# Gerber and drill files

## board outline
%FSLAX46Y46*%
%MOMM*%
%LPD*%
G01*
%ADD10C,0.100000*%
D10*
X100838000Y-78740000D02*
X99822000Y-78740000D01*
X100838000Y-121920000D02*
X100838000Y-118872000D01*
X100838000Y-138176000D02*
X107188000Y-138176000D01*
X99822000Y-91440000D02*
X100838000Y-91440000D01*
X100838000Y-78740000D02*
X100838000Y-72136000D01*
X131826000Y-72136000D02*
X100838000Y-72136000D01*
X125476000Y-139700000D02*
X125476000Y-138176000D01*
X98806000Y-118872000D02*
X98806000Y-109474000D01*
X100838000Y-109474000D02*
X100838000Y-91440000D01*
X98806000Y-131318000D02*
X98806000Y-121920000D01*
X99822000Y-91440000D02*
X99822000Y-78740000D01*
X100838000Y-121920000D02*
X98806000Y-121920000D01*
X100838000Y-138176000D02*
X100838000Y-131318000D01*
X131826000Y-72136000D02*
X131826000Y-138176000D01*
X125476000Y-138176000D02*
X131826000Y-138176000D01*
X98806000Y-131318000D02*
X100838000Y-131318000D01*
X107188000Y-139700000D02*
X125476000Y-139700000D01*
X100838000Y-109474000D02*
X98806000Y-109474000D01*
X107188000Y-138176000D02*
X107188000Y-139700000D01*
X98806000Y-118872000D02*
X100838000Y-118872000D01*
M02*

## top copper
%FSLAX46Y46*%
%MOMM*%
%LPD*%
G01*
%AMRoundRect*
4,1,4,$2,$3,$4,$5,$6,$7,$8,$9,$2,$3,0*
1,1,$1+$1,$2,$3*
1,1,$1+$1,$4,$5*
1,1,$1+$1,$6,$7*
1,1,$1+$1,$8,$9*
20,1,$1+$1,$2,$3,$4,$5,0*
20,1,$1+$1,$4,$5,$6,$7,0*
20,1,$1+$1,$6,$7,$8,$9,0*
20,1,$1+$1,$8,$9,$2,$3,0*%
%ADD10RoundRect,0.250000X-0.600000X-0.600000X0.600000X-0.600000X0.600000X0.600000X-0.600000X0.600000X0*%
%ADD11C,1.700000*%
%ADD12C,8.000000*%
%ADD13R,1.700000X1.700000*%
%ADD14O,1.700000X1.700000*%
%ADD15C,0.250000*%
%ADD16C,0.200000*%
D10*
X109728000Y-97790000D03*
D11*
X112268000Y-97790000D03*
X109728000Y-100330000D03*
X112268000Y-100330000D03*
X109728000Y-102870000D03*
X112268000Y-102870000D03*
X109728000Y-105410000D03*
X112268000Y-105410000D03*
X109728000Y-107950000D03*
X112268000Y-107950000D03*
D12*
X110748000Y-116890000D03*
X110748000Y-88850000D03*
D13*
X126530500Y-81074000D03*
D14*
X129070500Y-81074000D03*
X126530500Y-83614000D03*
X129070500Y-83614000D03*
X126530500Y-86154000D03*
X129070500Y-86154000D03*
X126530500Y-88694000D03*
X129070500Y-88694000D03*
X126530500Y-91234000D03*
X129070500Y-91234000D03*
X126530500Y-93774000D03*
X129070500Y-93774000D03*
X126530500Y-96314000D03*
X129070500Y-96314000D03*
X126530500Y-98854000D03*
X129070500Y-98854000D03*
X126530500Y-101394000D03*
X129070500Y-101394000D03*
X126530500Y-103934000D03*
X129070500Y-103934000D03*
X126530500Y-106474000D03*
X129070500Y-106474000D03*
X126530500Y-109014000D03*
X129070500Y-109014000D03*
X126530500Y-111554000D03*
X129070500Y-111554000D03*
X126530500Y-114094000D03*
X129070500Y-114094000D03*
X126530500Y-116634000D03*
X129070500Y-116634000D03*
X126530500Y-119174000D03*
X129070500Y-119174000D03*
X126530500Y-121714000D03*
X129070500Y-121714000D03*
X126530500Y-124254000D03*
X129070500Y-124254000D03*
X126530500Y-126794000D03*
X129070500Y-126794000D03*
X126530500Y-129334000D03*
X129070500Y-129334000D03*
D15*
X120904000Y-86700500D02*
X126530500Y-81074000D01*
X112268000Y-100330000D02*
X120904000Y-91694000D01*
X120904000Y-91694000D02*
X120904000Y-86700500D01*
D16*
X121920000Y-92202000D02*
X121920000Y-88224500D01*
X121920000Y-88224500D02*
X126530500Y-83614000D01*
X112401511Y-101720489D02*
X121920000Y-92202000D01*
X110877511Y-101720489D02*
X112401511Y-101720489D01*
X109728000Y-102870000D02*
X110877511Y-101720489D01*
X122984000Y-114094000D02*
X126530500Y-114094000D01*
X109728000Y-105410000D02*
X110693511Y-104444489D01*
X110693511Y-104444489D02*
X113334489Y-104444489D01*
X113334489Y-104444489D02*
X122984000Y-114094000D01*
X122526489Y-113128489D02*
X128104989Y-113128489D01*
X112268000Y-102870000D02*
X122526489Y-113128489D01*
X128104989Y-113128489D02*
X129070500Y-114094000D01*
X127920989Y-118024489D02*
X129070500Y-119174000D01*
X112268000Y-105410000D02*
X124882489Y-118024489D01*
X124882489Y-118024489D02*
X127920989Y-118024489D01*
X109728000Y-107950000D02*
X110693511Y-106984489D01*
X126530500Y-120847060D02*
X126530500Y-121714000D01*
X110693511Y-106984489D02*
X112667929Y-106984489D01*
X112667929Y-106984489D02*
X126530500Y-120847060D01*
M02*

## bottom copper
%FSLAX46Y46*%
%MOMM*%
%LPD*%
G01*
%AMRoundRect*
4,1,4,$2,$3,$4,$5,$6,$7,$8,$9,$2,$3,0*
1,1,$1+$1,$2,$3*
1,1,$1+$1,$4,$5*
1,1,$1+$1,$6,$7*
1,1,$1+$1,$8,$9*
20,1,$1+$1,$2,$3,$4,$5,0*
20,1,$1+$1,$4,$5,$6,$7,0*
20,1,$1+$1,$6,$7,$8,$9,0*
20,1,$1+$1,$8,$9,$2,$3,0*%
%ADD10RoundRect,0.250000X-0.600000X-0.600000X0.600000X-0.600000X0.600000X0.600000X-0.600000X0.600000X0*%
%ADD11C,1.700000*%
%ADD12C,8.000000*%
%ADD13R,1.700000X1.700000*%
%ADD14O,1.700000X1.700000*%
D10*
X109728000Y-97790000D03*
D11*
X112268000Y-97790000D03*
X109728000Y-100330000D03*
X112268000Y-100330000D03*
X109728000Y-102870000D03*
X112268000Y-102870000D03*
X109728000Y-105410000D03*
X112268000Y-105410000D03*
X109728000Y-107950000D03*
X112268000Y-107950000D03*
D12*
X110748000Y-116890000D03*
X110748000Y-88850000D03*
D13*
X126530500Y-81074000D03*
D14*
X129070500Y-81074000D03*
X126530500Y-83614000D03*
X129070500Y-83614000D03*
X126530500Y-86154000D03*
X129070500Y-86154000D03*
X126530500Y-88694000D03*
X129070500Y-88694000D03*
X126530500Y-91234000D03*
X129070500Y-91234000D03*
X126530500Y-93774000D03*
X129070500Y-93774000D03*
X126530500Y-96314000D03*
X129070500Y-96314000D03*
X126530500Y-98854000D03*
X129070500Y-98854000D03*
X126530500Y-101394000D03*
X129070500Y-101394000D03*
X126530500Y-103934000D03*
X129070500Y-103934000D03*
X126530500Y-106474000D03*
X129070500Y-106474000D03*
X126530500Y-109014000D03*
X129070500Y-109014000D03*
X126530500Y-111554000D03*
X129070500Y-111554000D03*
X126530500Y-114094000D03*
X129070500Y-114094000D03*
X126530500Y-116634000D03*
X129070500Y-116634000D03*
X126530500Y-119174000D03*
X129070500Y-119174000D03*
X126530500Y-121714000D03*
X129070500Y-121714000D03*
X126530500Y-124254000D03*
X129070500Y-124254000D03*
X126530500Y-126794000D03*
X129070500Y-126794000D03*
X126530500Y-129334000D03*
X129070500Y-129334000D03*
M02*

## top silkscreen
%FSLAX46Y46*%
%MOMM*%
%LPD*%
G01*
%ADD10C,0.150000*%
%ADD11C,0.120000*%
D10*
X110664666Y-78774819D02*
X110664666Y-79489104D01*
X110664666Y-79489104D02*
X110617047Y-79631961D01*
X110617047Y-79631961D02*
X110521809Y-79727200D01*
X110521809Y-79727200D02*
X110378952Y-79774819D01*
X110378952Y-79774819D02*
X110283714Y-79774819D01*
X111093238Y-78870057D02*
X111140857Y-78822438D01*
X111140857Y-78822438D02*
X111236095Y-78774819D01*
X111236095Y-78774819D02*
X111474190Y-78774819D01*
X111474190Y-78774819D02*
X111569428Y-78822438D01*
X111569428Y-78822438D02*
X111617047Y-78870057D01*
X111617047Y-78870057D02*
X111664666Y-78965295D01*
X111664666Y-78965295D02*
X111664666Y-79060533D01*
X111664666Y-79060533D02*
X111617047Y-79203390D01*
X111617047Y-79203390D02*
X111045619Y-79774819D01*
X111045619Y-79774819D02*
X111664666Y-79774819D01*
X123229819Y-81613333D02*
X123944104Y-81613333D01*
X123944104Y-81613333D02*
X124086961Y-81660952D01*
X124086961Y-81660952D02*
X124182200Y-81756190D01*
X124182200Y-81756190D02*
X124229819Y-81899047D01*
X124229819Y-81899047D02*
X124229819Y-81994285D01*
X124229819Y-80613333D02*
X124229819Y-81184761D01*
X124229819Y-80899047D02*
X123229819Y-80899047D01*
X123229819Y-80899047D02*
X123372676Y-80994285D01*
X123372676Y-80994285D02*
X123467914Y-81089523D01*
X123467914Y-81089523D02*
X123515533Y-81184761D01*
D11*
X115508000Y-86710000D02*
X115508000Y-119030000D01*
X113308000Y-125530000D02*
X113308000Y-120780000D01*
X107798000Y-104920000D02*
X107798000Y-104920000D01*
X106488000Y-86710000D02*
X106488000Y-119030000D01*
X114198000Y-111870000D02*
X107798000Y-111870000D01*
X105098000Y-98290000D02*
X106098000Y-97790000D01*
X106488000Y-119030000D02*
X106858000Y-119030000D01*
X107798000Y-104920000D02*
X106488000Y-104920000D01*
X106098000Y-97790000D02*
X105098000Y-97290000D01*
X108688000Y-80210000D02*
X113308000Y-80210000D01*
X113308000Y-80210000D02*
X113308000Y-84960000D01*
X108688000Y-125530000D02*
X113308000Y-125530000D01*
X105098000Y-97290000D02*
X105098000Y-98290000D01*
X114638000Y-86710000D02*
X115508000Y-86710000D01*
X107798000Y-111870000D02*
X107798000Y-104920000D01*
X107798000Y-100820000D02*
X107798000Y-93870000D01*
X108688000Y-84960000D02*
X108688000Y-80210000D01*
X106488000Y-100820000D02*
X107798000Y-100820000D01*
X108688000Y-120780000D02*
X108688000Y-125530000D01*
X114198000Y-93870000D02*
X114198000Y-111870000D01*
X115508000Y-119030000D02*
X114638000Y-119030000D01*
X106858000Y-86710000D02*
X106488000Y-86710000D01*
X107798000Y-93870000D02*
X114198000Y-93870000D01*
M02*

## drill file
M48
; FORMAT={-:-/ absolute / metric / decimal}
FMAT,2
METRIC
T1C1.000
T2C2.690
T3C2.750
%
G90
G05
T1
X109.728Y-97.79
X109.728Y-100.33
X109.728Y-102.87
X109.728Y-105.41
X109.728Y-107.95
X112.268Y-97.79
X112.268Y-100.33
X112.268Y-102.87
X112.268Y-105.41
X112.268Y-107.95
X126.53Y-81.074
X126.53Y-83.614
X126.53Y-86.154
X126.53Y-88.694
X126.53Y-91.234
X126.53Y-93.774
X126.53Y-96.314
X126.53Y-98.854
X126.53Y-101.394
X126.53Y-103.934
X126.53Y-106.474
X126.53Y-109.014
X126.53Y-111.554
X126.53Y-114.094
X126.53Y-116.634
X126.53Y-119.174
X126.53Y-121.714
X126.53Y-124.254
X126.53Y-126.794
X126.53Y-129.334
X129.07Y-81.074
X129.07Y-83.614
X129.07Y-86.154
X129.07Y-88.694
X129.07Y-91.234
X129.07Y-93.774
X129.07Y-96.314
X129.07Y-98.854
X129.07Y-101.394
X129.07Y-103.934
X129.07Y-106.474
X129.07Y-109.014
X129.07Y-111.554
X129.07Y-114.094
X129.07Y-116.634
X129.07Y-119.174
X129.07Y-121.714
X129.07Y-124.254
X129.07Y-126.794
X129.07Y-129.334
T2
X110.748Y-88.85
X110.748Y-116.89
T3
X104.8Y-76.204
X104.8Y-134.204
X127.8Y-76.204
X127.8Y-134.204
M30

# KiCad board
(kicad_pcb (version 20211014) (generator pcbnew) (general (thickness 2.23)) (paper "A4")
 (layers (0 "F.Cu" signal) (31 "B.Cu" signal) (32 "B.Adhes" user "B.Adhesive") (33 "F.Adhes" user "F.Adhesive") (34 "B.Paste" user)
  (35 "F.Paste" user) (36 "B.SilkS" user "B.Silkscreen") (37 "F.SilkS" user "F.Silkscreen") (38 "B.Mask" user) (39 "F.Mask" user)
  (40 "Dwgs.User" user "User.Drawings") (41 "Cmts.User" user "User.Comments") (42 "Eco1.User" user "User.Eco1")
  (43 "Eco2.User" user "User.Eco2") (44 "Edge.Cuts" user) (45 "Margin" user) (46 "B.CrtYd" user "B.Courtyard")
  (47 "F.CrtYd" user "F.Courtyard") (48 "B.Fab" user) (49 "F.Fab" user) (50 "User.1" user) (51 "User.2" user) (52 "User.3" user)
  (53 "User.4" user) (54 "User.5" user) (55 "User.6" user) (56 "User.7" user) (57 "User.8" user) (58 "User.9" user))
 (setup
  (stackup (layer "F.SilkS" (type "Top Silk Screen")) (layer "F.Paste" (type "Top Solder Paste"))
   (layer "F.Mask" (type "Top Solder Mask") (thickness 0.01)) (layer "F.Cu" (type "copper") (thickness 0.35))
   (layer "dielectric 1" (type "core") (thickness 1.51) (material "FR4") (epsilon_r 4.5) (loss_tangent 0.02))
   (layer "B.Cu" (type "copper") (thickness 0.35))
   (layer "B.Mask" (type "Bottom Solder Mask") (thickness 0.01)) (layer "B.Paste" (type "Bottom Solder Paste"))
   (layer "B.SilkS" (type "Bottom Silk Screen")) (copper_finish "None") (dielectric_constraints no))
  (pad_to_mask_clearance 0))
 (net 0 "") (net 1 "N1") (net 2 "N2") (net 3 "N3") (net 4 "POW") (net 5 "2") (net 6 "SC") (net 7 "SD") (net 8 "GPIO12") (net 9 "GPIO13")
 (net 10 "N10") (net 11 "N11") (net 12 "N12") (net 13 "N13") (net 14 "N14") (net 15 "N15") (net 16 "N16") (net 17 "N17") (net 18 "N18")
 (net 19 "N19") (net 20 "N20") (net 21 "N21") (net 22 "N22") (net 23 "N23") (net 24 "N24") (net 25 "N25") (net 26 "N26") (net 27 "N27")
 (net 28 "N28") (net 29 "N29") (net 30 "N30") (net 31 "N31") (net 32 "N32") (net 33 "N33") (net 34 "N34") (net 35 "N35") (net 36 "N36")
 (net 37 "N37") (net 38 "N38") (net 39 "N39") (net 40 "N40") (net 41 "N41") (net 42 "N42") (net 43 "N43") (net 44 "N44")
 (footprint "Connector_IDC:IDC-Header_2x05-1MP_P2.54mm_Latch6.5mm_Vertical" (layer "F.Cu") (at 109.728 97.79)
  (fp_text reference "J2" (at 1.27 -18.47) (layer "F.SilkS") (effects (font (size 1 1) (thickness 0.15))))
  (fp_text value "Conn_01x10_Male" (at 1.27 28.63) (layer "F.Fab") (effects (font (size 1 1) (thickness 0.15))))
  (fp_line (start 5.78 -11.08) (end 5.78 21.24) (layer "F.SilkS") (width 0.12))
  (fp_line (start 3.58 27.74) (end 3.58 22.99) (layer "F.SilkS") (width 0.12))
  (fp_line (start -1.93 7.13) (end -1.93 7.13) (layer "F.SilkS") (width 0.12))
  (fp_line (start -3.24 -11.08) (end -3.24 21.24) (layer "F.SilkS") (width 0.12))
  (fp_line (start 4.47 14.08) (end -1.93 14.08) (layer "F.SilkS") (width 0.12))
  (fp_line (start -4.63 0.5) (end -3.63 0) (layer "F.SilkS") (width 0.12))
  (fp_line (start -3.24 21.24) (end -2.87 21.24) (layer "F.SilkS") (width 0.12))
  (fp_line (start -1.93 7.13) (end -3.24 7.13) (layer "F.SilkS") (width 0.12))
  (fp_line (start -3.63 0) (end -4.63 -0.5) (layer "F.SilkS") (width 0.12))
  (fp_line (start -1.04 -17.58) (end 3.58 -17.58) (layer "F.SilkS") (width 0.12))
  (fp_line (start 3.58 -17.58) (end 3.58 -12.83) (layer "F.SilkS") (width 0.12))
  (fp_line (start -1.04 27.74) (end 3.58 27.74) (layer "F.SilkS") (width 0.12))
  (fp_line (start -4.63 -0.5) (end -4.63 0.5) (layer "F.SilkS") (width 0.12))
  (fp_line (start 4.91 -11.08) (end 5.78 -11.08) (layer "F.SilkS") (width 0.12))
  (fp_line (start -1.93 14.08) (end -1.93 7.13) (layer "F.SilkS") (width 0.12))
  (fp_line (start -1.93 3.03) (end -1.93 -3.92) (layer "F.SilkS") (width 0.12))
  (fp_line (start -1.04 -12.83) (end -1.04 -17.58) (layer "F.SilkS") (width 0.12))
  (fp_line (start -3.24 3.03) (end -1.93 3.03) (layer "F.SilkS") (width 0.12))
  (fp_line (start -1.04 22.99) (end -1.04 27.74) (layer "F.SilkS") (width 0.12))
  (fp_line (start 4.47 -3.92) (end 4.47 14.08) (layer "F.SilkS") (width 0.12))
  (fp_line (start 5.78 21.24) (end 4.91 21.24) (layer "F.SilkS") (width 0.12))
  (fp_line (start -2.87 -11.08) (end -3.24 -11.08) (layer "F.SilkS") (width 0.12))
  (fp_line (start -1.93 -3.92) (end 4.47 -3.92) (layer "F.SilkS") (width 0.12))
  (pad "1" thru_hole roundrect (at 0 0) (size 1.7 1.7) (drill 1) (layers *.Cu *.Mask) (roundrect_rratio 0.147059) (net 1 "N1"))
  (pad "2" thru_hole circle (at 2.54 0) (size 1.7 1.7) (drill 1) (layers *.Cu *.Mask) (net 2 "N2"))
  (pad "3" thru_hole circle (at 0 2.54) (size 1.7 1.7) (drill 1) (layers *.Cu *.Mask) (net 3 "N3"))
  (pad "4" thru_hole circle (at 2.54 2.54) (size 1.7 1.7) (drill 1) (layers *.Cu *.Mask) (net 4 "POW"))
  (pad "5" thru_hole circle (at 0 5.08) (size 1.7 1.7) (drill 1) (layers *.Cu *.Mask) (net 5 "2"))
  (pad "6" thru_hole circle (at 2.54 5.08) (size 1.7 1.7) (drill 1) (layers *.Cu *.Mask) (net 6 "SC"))
  (pad "7" thru_hole circle (at 0 7.62) (size 1.7 1.7) (drill 1) (layers *.Cu *.Mask) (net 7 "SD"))
  (pad "8" thru_hole circle (at 2.54 7.62) (size 1.7 1.7) (drill 1) (layers *.Cu *.Mask) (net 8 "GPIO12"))
  (pad "9" thru_hole circle (at 0 10.16) (size 1.7 1.7) (drill 1) (layers *.Cu *.Mask) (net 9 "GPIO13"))
  (pad "10" thru_hole circle (at 2.54 10.16) (size 1.7 1.7) (drill 1) (layers *.Cu *.Mask) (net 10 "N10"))
  (pad "MP" thru_hole circle (at 1.02 19.1) (size 8 8) (drill 2.69) (layers *.Cu *.Mask))
  (pad "MP" thru_hole circle (at 1.02 -8.94) (size 8 8) (drill 2.69) (layers *.Cu *.Mask)))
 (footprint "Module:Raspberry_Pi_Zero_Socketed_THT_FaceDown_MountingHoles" (layer "B.Cu") (at 126.5305 81.074 180)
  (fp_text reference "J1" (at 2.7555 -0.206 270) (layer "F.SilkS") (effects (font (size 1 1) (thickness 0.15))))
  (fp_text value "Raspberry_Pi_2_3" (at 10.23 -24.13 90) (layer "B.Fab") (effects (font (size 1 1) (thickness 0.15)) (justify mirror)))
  (pad "" np_thru_hole circle (at 21.73 4.87 90) (size 2.75 2.75) (drill 2.75) (layers *.Cu *.Mask) (solder_mask_margin 1.625))
  (pad "" np_thru_hole circle (at 21.73 -53.13 90) (size 2.75 2.75) (drill 2.75) (layers *.Cu *.Mask) (solder_mask_margin 1.625))
  (pad "" np_thru_hole circle (at -1.27 4.87 90) (size 2.75 2.75) (drill 2.75) (layers *.Cu *.Mask) (solder_mask_margin 1.625))
  (pad "" np_thru_hole circle (at -1.27 -53.13 90) (size 2.75 2.75) (drill 2.75) (layers *.Cu *.Mask) (solder_mask_margin 1.625))
  (pad "1" thru_hole rect (at 0 0 180) (size 1.7 1.7) (drill 1) (layers *.Cu *.Mask) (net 4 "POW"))
  (pad "2" thru_hole oval (at -2.54 0 180) (size 1.7 1.7) (drill 1) (layers *.Cu *.Mask) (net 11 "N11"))
  (pad "3" thru_hole oval (at 0 -2.54 180) (size 1.7 1.7) (drill 1) (layers *.Cu *.Mask) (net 5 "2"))
  (pad "4" thru_hole oval (at -2.54 -2.54 180) (size 1.7 1.7) (drill 1) (layers *.Cu *.Mask) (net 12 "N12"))
  (pad "5" thru_hole oval (at 0 -5.08 180) (size 1.7 1.7) (drill 1) (layers *.Cu *.Mask) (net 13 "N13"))
  (pad "6" thru_hole oval (at -2.54 -5.08 180) (size 1.7 1.7) (drill 1) (layers *.Cu *.Mask) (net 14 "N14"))
  (pad "7" thru_hole oval (at 0 -7.62 180) (size 1.7 1.7) (drill 1) (layers *.Cu *.Mask) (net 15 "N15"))
  (pad "8" thru_hole oval (at -2.54 -7.62 180) (size 1.7 1.7) (drill 1) (layers *.Cu *.Mask) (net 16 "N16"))
  (pad "9" thru_hole oval (at 0 -10.16 180) (size 1.7 1.7) (drill 1) (layers *.Cu *.Mask) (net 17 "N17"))
  (pad "10" thru_hole oval (at -2.54 -10.16 180) (size 1.7 1.7) (drill 1) (layers *.Cu *.Mask) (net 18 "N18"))
  (pad "11" thru_hole oval (at 0 -12.7 180) (size 1.7 1.7) (drill 1) (layers *.Cu *.Mask) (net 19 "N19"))
  (pad "12" thru_hole oval (at -2.54 -12.7 180) (size 1.7 1.7) (drill 1) (layers *.Cu *.Mask) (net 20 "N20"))
  (pad "13" thru_hole oval (at 0 -15.24 180) (size 1.7 1.7) (drill 1) (layers *.Cu *.Mask) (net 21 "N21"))
  (pad "14" thru_hole oval (at -2.54 -15.24 180) (size 1.7 1.7) (drill 1) (layers *.Cu *.Mask) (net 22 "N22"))
  (pad "15" thru_hole oval (at 0 -17.78 180) (size 1.7 1.7) (drill 1) (layers *.Cu *.Mask) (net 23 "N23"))
  (pad "16" thru_hole oval (at -2.54 -17.78 180) (size 1.7 1.7) (drill 1) (layers *.Cu *.Mask) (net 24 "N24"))
  (pad "17" thru_hole oval (at 0 -20.32 180) (size 1.7 1.7) (drill 1) (layers *.Cu *.Mask) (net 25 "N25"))
  (pad "18" thru_hole oval (at -2.54 -20.32 180) (size 1.7 1.7) (drill 1) (layers *.Cu *.Mask) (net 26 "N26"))
  (pad "19" thru_hole oval (at 0 -22.86 180) (size 1.7 1.7) (drill 1) (layers *.Cu *.Mask) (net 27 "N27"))
  (pad "20" thru_hole oval (at -2.54 -22.86 180) (size 1.7 1.7) (drill 1) (layers *.Cu *.Mask) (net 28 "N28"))
  (pad "21" thru_hole oval (at 0 -25.4 180) (size 1.7 1.7) (drill 1) (layers *.Cu *.Mask) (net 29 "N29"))
  (pad "22" thru_hole oval (at -2.54 -25.4 180) (size 1.7 1.7) (drill 1) (layers *.Cu *.Mask) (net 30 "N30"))
  (pad "23" thru_hole oval (at 0 -27.94 180) (size 1.7 1.7) (drill 1) (layers *.Cu *.Mask) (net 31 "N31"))
  (pad "24" thru_hole oval (at -2.54 -27.94 180) (size 1.7 1.7) (drill 1) (layers *.Cu *.Mask) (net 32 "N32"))
  (pad "25" thru_hole oval (at 0 -30.48 180) (size 1.7 1.7) (drill 1) (layers *.Cu *.Mask) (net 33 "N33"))
  (pad "26" thru_hole oval (at -2.54 -30.48 180) (size 1.7 1.7) (drill 1) (layers *.Cu *.Mask) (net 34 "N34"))
  (pad "27" thru_hole oval (at 0 -33.02 180) (size 1.7 1.7) (drill 1) (layers *.Cu *.Mask) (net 7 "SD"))
  (pad "28" thru_hole oval (at -2.54 -33.02 180) (size 1.7 1.7) (drill 1) (layers *.Cu *.Mask) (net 6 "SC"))
  (pad "29" thru_hole oval (at 0 -35.56 180) (size 1.7 1.7) (drill 1) (layers *.Cu *.Mask) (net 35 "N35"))
  (pad "30" thru_hole oval (at -2.54 -35.56 180) (size 1.7 1.7) (drill 1) (layers *.Cu *.Mask) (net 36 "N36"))
  (pad "31" thru_hole oval (at 0 -38.1 180) (size 1.7 1.7) (drill 1) (layers *.Cu *.Mask) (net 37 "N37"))
  (pad "32" thru_hole oval (at -2.54 -38.1 180) (size 1.7 1.7) (drill 1) (layers *.Cu *.Mask) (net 8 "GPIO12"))
  (pad "33" thru_hole oval (at 0 -40.64 180) (size 1.7 1.7) (drill 1) (layers *.Cu *.Mask) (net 9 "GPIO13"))
  (pad "34" thru_hole oval (at -2.54 -40.64 180) (size 1.7 1.7) (drill 1) (layers *.Cu *.Mask) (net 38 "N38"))
  (pad "35" thru_hole oval (at 0 -43.18 180) (size 1.7 1.7) (drill 1) (layers *.Cu *.Mask) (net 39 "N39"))
  (pad "36" thru_hole oval (at -2.54 -43.18 180) (size 1.7 1.7) (drill 1) (layers *.Cu *.Mask) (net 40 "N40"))
  (pad "37" thru_hole oval (at 0 -45.72 180) (size 1.7 1.7) (drill 1) (layers *.Cu *.Mask) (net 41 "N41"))
  (pad "38" thru_hole oval (at -2.54 -45.72 180) (size 1.7 1.7) (drill 1) (layers *.Cu *.Mask) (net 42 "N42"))
  (pad "39" thru_hole oval (at 0 -48.26 180) (size 1.7 1.7) (drill 1) (layers *.Cu *.Mask) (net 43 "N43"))
  (pad "40" thru_hole oval (at -2.54 -48.26 180) (size 1.7 1.7) (drill 1) (layers *.Cu *.Mask) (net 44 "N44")))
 (gr_line (start 100.838 78.74) (end 99.822 78.74) (layer "Edge.Cuts") (width 0.1))
 (gr_line (start 100.838 121.92) (end 100.838 118.872) (layer "Edge.Cuts") (width 0.1))
 (gr_line (start 100.838 138.176) (end 107.188 138.176) (layer "Edge.Cuts") (width 0.1))
 (gr_line (start 99.822 91.44) (end 100.838 91.44) (layer "Edge.Cuts") (width 0.1))
 (gr_line (start 100.838 78.74) (end 100.838 72.136) (layer "Edge.Cuts") (width 0.1))
 (gr_line (start 131.826 72.136) (end 100.838 72.136) (layer "Edge.Cuts") (width 0.1))
 (gr_line (start 125.476 139.7) (end 125.476 138.176) (layer "Edge.Cuts") (width 0.1))
 (gr_line (start 98.806 118.872) (end 98.806 109.474) (layer "Edge.Cuts") (width 0.1))
 (gr_line (start 100.838 109.474) (end 100.838 91.44) (layer "Edge.Cuts") (width 0.1))
 (gr_line (start 98.806 131.318) (end 98.806 121.92) (layer "Edge.Cuts") (width 0.1))
 (gr_line (start 99.822 91.44) (end 99.822 78.74) (layer "Edge.Cuts") (width 0.1))
 (gr_line (start 100.838 121.92) (end 98.806 121.92) (layer "Edge.Cuts") (width 0.1))
 (gr_line (start 100.838 138.176) (end 100.838 131.318) (layer "Edge.Cuts") (width 0.1))
 (gr_line (start 131.826 72.136) (end 131.826 138.176) (layer "Edge.Cuts") (width 0.1))
 (gr_line (start 125.476 138.176) (end 131.826 138.176) (layer "Edge.Cuts") (width 0.1))
 (gr_line (start 98.806 131.318) (end 100.838 131.318) (layer "Edge.Cuts") (width 0.1))
 (gr_line (start 107.188 139.7) (end 125.476 139.7) (layer "Edge.Cuts") (width 0.1))
 (gr_line (start 100.838 109.474) (end 98.806 109.474) (layer "Edge.Cuts") (width 0.1))
 (gr_line (start 107.188 138.176) (end 107.188 139.7) (layer "Edge.Cuts") (width 0.1))
 (gr_line (start 98.806 118.872) (end 100.838 118.872) (layer "Edge.Cuts") (width 0.1))
 (segment (start 120.904 86.7005) (end 126.5305 81.074) (width 0.25) (layer "F.Cu") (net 4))
 (segment (start 112.268 100.33) (end 120.904 91.694) (width 0.25) (layer "F.Cu") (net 4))
 (segment (start 120.904 91.694) (end 120.904 86.7005) (width 0.25) (layer "F.Cu") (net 4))
 (segment (start 121.92 92.202) (end 121.92 88.2245) (width 0.2) (layer "F.Cu") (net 5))
 (segment (start 121.92 88.2245) (end 126.5305 83.614) (width 0.2) (layer "F.Cu") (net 5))
 (segment (start 112.401511 101.720489) (end 121.92 92.202) (width 0.2) (layer "F.Cu") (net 5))
 (segment (start 110.877511 101.720489) (end 112.401511 101.720489) (width 0.2) (layer "F.Cu") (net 5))
 (segment (start 109.728 102.87) (end 110.877511 101.720489) (width 0.2) (layer "F.Cu") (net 5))
 (segment (start 122.984 114.094) (end 126.5305 114.094) (width 0.2) (layer "F.Cu") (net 7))
 (segment (start 109.728 105.41) (end 110.693511 104.444489) (width 0.2) (layer "F.Cu") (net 7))
 (segment (start 110.693511 104.444489) (end 113.334489 104.444489) (width 0.2) (layer "F.Cu") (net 7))
 (segment (start 113.334489 104.444489) (end 122.984 114.094) (width 0.2) (layer "F.Cu") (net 7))
 (segment (start 122.526489 113.128489) (end 128.104989 113.128489) (width 0.2) (layer "F.Cu") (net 6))
 (segment (start 112.268 102.87) (end 122.526489 113.128489) (width 0.2) (layer "F.Cu") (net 6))
 (segment (start 128.104989 113.128489) (end 129.0705 114.094) (width 0.2) (layer "F.Cu") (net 6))
 (segment (start 127.920989 118.024489) (end 129.0705 119.174) (width 0.2) (layer "F.Cu") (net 8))
 (segment (start 112.268 105.41) (end 124.882489 118.024489) (width 0.2) (layer "F.Cu") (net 8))
 (segment (start 124.882489 118.024489) (end 127.920989 118.024489) (width 0.2) (layer "F.Cu") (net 8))
 (segment (start 109.728 107.95) (end 110.693511 106.984489) (width 0.2) (layer "F.Cu") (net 9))
 (segment (start 126.5305 120.84706) (end 126.5305 121.714) (width 0.2) (layer "F.Cu") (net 9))
 (segment (start 110.693511 106.984489) (end 112.667929 106.984489) (width 0.2) (layer "F.Cu") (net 9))
 (segment (start 112.667929 106.984489) (end 126.5305 120.84706) (width 0.2) (layer "F.Cu") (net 9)))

